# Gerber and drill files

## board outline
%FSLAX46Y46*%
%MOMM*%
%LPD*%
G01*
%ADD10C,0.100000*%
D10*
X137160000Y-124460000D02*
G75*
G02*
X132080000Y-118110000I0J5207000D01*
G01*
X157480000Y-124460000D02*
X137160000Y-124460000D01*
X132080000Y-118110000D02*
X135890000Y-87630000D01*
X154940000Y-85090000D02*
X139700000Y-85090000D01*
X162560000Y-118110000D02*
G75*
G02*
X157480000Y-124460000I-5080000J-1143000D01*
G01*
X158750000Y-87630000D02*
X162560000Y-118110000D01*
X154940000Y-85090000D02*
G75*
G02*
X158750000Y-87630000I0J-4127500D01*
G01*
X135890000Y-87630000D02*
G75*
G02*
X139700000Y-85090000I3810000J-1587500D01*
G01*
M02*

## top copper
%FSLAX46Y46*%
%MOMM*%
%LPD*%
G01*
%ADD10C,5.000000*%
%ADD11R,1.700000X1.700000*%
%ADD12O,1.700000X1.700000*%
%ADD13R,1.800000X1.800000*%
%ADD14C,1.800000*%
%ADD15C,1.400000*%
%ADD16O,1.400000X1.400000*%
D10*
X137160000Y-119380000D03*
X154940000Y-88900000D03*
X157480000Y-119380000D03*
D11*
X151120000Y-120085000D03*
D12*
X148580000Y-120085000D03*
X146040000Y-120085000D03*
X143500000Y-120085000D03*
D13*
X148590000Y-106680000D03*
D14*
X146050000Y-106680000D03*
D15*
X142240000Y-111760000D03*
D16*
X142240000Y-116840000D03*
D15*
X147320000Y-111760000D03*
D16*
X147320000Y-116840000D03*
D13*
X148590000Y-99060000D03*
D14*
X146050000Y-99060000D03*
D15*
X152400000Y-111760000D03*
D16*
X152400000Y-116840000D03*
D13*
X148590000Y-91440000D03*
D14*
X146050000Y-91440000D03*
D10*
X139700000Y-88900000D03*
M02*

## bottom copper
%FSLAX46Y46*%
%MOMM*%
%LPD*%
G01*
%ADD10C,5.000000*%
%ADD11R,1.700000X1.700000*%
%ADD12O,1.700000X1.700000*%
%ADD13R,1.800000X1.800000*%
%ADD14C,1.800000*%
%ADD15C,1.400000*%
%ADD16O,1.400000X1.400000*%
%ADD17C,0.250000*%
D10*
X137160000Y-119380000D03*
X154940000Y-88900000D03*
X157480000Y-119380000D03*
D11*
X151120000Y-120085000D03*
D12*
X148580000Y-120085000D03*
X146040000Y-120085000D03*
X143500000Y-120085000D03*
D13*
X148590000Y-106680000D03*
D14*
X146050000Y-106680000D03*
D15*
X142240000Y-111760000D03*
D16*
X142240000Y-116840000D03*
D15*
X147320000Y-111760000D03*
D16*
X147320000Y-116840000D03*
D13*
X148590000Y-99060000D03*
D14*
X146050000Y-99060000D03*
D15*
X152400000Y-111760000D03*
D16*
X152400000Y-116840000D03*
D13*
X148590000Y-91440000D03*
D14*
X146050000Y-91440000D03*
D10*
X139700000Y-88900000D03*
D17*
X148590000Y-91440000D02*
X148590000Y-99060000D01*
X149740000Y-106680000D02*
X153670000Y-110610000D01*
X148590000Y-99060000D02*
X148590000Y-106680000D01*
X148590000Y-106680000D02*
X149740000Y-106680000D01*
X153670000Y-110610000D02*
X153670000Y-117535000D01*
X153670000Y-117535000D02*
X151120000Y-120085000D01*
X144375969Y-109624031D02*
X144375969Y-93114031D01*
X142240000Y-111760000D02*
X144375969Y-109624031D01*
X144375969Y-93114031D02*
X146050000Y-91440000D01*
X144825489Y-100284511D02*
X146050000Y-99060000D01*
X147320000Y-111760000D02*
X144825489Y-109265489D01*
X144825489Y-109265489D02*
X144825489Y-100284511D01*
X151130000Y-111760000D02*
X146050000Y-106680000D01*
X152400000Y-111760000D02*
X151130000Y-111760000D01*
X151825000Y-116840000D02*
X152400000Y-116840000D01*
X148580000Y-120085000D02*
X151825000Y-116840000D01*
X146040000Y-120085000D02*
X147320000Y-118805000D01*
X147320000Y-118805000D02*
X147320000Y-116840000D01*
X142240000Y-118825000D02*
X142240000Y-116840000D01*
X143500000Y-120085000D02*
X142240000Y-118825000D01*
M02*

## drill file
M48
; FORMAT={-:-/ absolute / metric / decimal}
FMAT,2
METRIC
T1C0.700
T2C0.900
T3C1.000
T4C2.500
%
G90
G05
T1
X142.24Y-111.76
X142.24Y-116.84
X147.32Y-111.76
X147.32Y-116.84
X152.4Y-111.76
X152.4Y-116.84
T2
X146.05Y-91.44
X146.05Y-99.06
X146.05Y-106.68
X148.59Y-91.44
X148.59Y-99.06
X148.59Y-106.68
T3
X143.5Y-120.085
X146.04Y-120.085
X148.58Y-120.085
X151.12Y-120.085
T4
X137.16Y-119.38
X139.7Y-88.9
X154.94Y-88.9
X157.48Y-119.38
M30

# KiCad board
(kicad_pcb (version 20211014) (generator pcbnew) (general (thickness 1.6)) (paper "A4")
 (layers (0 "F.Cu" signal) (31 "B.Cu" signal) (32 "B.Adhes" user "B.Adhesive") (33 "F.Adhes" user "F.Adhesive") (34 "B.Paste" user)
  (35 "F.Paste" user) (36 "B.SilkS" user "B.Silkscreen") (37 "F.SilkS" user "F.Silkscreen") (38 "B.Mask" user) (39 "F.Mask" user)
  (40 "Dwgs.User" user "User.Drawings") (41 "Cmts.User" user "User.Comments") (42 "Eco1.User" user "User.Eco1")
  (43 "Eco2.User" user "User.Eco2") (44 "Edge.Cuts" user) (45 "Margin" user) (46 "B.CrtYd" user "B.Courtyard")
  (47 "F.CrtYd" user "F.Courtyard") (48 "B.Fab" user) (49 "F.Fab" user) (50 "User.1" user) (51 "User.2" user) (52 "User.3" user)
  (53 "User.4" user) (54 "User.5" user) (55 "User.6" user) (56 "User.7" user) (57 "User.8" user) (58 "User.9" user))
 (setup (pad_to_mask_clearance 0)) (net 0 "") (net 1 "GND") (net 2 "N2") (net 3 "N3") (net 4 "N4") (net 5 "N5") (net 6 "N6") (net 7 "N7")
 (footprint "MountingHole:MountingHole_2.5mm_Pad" (layer "F.Cu") (at 137.16 119.38)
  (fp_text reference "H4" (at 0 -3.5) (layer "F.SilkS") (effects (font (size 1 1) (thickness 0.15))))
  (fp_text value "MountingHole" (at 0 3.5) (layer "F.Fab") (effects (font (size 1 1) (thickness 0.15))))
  (pad "1" thru_hole circle (at 0 0) (size 5 5) (drill 2.5) (layers *.Cu *.Mask)))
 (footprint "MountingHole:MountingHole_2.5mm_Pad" (layer "F.Cu") (at 154.94 88.9 180)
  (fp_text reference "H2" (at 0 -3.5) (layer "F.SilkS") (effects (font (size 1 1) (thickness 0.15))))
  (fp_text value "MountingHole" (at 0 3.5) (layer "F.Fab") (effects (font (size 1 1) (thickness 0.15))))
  (pad "1" thru_hole circle (at 0 0 180) (size 5 5) (drill 2.5) (layers *.Cu *.Mask)))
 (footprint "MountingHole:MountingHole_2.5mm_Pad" (layer "F.Cu") (at 157.48 119.38)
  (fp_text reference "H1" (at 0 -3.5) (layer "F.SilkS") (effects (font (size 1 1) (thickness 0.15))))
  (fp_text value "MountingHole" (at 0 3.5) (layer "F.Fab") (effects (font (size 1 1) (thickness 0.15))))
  (pad "1" thru_hole circle (at 0 0) (size 5 5) (drill 2.5) (layers *.Cu *.Mask)))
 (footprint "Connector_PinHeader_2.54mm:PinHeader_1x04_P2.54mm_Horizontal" (layer "F.Cu") (at 151.12 120.085 -90)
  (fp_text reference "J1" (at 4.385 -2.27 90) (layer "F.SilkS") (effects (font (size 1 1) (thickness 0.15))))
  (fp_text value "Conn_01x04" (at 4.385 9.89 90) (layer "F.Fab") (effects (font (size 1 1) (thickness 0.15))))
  (pad "1" thru_hole rect (at 0 0 270) (size 1.7 1.7) (drill 1) (layers *.Cu *.Mask) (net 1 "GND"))
  (pad "2" thru_hole oval (at 0 2.54 270) (size 1.7 1.7) (drill 1) (layers *.Cu *.Mask) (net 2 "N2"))
  (pad "3" thru_hole oval (at 0 5.08 270) (size 1.7 1.7) (drill 1) (layers *.Cu *.Mask) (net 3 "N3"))
  (pad "4" thru_hole oval (at 0 7.62 270) (size 1.7 1.7) (drill 1) (layers *.Cu *.Mask) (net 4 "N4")))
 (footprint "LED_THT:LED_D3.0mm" (layer "F.Cu") (at 148.59 106.68 180)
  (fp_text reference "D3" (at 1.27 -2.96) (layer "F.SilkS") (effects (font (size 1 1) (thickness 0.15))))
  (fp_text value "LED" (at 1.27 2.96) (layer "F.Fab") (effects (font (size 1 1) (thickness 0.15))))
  (pad "1" thru_hole rect (at 0 0 180) (size 1.8 1.8) (drill 0.9) (layers *.Cu *.Mask) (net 1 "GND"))
  (pad "2" thru_hole circle (at 2.54 0 180) (size 1.8 1.8) (drill 0.9) (layers *.Cu *.Mask) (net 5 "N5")))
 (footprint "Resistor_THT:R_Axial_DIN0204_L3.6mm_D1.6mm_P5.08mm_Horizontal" (layer "F.Cu") (at 142.24 111.76 -90)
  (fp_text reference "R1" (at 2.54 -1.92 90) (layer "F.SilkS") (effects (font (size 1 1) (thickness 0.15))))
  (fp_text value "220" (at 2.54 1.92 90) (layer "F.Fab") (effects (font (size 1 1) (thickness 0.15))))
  (pad "1" thru_hole circle (at 0 0 270) (size 1.4 1.4) (drill 0.7) (layers *.Cu *.Mask) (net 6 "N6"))
  (pad "2" thru_hole oval (at 5.08 0 270) (size 1.4 1.4) (drill 0.7) (layers *.Cu *.Mask) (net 4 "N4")))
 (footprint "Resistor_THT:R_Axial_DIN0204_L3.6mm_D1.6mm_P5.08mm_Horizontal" (layer "F.Cu") (at 147.32 111.76 -90)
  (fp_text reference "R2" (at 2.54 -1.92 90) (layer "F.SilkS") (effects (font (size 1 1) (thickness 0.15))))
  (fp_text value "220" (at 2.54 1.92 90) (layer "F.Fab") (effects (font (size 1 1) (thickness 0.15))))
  (pad "1" thru_hole circle (at 0 0 270) (size 1.4 1.4) (drill 0.7) (layers *.Cu *.Mask) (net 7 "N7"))
  (pad "2" thru_hole oval (at 5.08 0 270) (size 1.4 1.4) (drill 0.7) (layers *.Cu *.Mask) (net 3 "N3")))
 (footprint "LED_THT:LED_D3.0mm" (layer "F.Cu") (at 148.59 99.06 180)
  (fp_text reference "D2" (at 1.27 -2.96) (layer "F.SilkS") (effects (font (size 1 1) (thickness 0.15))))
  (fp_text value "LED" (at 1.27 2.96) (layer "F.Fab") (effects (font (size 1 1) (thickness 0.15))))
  (pad "1" thru_hole rect (at 0 0 180) (size 1.8 1.8) (drill 0.9) (layers *.Cu *.Mask) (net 1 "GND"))
  (pad "2" thru_hole circle (at 2.54 0 180) (size 1.8 1.8) (drill 0.9) (layers *.Cu *.Mask) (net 7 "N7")))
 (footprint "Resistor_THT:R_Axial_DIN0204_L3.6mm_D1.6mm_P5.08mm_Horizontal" (layer "F.Cu") (at 152.4 111.76 -90)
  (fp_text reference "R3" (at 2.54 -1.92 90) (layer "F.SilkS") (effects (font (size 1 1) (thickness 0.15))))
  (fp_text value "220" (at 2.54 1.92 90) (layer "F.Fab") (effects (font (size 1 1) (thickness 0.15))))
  (pad "1" thru_hole circle (at 0 0 270) (size 1.4 1.4) (drill 0.7) (layers *.Cu *.Mask) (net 5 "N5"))
  (pad "2" thru_hole oval (at 5.08 0 270) (size 1.4 1.4) (drill 0.7) (layers *.Cu *.Mask) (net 2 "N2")))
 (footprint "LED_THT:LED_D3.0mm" (layer "F.Cu") (at 148.59 91.44 180)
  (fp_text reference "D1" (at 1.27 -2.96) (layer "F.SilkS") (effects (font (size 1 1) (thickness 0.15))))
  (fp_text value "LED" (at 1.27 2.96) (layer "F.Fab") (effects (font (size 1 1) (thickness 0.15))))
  (pad "1" thru_hole rect (at 0 0 180) (size 1.8 1.8) (drill 0.9) (layers *.Cu *.Mask) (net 1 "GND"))
  (pad "2" thru_hole circle (at 2.54 0 180) (size 1.8 1.8) (drill 0.9) (layers *.Cu *.Mask) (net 6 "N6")))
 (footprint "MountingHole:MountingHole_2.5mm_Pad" (layer "F.Cu") (at 139.7 88.9 180)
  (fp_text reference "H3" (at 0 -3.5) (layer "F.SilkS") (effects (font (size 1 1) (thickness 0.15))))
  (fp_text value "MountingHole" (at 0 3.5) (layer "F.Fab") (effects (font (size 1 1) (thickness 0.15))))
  (pad "1" thru_hole circle (at 0 0 180) (size 5 5) (drill 2.5) (layers *.Cu *.Mask)))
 (gr_arc (start 137.16 124.46) (mid 133.094016 122.505787) (end 132.08 118.11) (layer "Edge.Cuts") (width 0.1))
 (gr_line (start 157.48 124.46) (end 137.16 124.46) (layer "Edge.Cuts") (width 0.1))
 (gr_line (start 132.08 118.11) (end 135.89 87.63) (layer "Edge.Cuts") (width 0.1))
 (gr_line (start 154.94 85.09) (end 139.7 85.09) (layer "Edge.Cuts") (width 0.1))
 (gr_arc (start 162.56 118.11) (mid 161.545984 122.505787) (end 157.48 124.46) (layer "Edge.Cuts") (width 0.1))
 (gr_line (start 158.75 87.63) (end 162.56 118.11) (layer "Edge.Cuts") (width 0.1))
 (gr_arc (start 154.94 85.09) (mid 157.229525 85.783212) (end 158.75 87.63) (layer "Edge.Cuts") (width 0.1))
 (gr_arc (start 135.89 87.63) (mid 137.410475 85.783212) (end 139.7 85.09) (layer "Edge.Cuts") (width 0.1))
 (segment (start 148.59 91.44) (end 148.59 99.06) (width 0.25) (layer "B.Cu") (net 1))
 (segment (start 149.74 106.68) (end 153.67 110.61) (width 0.25) (layer "B.Cu") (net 1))
 (segment (start 148.59 99.06) (end 148.59 106.68) (width 0.25) (layer "B.Cu") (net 1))
 (segment (start 148.59 106.68) (end 149.74 106.68) (width 0.25) (layer "B.Cu") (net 1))
 (segment (start 153.67 110.61) (end 153.67 117.535) (width 0.25) (layer "B.Cu") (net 1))
 (segment (start 153.67 117.535) (end 151.12 120.085) (width 0.25) (layer "B.Cu") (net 1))
 (segment (start 144.375969 109.624031) (end 144.375969 93.114031) (width 0.25) (layer "B.Cu") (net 6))
 (segment (start 142.24 111.76) (end 144.375969 109.624031) (width 0.25) (layer "B.Cu") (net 6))
 (segment (start 144.375969 93.114031) (end 146.05 91.44) (width 0.25) (layer "B.Cu") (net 6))
 (segment (start 144.825489 100.284511) (end 146.05 99.06) (width 0.25) (layer "B.Cu") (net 7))
 (segment (start 147.32 111.76) (end 144.825489 109.265489) (width 0.25) (layer "B.Cu") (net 7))
 (segment (start 144.825489 109.265489) (end 144.825489 100.284511) (width 0.25) (layer "B.Cu") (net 7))
 (segment (start 151.13 111.76) (end 146.05 106.68) (width 0.25) (layer "B.Cu") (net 5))
 (segment (start 152.4 111.76) (end 151.13 111.76) (width 0.25) (layer "B.Cu") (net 5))
 (segment (start 151.825 116.84) (end 152.4 116.84) (width 0.25) (layer "B.Cu") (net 2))
 (segment (start 148.58 120.085) (end 151.825 116.84) (width 0.25) (layer "B.Cu") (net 2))
 (segment (start 146.04 120.085) (end 147.32 118.805) (width 0.25) (layer "B.Cu") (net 3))
 (segment (start 147.32 118.805) (end 147.32 116.84) (width 0.25) (layer "B.Cu") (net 3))
 (segment (start 142.24 118.825) (end 142.24 116.84) (width 0.25) (layer "B.Cu") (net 4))
 (segment (start 143.5 120.085) (end 142.24 118.825) (width 0.25) (layer "B.Cu") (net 4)))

